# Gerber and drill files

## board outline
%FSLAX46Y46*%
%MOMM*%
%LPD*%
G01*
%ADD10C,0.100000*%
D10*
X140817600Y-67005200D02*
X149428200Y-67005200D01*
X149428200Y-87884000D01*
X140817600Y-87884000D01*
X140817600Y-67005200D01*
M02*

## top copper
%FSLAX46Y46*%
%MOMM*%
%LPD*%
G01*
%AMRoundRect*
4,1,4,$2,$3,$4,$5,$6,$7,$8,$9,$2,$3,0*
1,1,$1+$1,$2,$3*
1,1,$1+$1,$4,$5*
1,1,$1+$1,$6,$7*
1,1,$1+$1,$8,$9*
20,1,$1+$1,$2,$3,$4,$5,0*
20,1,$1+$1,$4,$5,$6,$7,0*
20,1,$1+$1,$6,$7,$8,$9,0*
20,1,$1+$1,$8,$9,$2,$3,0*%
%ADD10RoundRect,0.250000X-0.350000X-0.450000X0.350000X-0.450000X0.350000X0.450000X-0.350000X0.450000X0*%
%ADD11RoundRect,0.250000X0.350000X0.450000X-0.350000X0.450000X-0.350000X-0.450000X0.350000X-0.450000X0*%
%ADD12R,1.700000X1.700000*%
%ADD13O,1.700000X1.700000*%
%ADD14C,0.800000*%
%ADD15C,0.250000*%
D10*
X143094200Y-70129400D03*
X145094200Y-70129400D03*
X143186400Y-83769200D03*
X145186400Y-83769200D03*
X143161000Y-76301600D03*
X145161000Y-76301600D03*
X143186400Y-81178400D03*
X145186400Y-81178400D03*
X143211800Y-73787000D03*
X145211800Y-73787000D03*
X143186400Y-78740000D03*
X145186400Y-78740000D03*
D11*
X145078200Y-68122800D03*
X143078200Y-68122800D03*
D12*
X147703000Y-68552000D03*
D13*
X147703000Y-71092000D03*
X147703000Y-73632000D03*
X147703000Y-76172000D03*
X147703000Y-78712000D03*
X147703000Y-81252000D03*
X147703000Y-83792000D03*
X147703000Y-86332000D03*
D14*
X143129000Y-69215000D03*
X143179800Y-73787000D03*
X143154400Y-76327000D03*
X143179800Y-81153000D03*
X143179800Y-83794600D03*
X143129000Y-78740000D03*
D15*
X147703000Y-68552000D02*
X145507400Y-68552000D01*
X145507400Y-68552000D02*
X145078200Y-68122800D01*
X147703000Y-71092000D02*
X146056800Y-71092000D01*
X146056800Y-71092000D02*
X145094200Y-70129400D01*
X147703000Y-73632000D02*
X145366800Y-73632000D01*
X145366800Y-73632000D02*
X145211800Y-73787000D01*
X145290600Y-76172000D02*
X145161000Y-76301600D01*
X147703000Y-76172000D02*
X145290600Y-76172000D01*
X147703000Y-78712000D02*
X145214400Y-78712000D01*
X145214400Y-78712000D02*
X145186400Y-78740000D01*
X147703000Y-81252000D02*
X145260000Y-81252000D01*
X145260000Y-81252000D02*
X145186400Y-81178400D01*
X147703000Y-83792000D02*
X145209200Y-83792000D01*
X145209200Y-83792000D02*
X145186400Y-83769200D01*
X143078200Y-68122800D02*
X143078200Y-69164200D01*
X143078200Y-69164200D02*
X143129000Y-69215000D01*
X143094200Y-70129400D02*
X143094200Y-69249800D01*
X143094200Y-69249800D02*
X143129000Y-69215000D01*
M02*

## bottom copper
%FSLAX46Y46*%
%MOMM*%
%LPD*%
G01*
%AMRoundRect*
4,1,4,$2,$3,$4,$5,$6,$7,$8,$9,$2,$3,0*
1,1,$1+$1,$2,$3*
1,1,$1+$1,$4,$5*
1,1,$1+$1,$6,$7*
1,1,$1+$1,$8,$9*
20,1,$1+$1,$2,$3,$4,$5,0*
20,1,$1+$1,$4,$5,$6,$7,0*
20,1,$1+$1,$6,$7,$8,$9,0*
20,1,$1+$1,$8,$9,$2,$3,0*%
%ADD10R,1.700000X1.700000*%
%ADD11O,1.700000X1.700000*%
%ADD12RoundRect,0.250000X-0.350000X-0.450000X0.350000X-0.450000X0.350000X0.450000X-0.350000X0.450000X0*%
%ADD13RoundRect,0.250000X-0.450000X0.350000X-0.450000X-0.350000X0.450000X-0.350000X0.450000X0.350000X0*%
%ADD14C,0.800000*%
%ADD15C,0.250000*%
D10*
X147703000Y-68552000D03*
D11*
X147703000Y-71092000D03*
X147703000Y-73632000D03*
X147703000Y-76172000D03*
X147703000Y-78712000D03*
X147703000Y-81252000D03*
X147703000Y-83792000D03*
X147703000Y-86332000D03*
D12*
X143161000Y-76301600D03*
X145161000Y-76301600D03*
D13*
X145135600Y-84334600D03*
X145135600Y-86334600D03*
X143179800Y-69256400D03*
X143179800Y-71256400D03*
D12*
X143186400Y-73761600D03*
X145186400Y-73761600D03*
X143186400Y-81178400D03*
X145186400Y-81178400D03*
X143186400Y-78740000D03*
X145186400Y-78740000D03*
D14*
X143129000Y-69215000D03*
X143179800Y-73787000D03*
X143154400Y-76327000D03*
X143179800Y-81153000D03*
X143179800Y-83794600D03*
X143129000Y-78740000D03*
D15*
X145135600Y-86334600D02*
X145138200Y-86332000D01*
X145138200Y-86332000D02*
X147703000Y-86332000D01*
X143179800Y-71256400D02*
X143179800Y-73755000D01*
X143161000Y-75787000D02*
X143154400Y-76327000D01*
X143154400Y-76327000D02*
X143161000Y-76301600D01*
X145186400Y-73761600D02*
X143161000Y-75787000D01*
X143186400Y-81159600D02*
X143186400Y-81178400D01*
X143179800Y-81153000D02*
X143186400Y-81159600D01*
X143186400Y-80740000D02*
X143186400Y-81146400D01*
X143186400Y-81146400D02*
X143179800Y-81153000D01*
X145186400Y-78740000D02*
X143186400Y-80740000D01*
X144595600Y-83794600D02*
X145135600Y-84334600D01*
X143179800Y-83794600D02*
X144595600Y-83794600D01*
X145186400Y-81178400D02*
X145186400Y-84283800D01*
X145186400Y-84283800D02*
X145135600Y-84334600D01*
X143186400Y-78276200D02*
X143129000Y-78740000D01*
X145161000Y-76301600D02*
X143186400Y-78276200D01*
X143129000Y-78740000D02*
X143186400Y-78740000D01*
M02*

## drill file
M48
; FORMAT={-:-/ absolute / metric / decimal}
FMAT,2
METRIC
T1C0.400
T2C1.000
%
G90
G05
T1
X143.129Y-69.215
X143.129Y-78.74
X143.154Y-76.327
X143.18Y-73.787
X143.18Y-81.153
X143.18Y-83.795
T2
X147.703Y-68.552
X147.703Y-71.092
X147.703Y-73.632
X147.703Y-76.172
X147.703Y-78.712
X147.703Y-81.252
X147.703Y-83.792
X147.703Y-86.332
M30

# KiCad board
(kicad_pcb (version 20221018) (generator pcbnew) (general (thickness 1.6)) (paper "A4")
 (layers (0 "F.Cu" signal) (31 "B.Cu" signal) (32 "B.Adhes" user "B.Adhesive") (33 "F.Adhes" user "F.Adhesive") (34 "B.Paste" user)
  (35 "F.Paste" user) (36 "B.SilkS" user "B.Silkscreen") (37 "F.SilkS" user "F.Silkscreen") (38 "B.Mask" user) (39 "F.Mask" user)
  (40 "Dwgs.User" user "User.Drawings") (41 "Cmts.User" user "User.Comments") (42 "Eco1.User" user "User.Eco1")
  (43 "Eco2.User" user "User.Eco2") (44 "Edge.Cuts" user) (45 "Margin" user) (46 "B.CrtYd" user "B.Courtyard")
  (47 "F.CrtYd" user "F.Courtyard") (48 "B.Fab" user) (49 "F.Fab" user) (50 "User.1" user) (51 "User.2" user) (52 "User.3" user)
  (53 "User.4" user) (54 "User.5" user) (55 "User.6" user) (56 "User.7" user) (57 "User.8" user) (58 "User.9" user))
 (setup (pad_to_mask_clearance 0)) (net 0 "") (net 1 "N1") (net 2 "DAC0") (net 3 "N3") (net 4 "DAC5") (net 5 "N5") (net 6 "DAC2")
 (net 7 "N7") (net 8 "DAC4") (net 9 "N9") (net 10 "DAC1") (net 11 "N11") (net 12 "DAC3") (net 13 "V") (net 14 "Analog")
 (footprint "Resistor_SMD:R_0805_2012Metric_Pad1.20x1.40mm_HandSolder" (layer "F.Cu") (at 144.0942 70.1294)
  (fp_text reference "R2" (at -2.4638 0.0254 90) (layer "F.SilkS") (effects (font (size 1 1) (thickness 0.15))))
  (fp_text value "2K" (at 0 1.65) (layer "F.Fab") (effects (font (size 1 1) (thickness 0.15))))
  (pad "1" smd roundrect (at -1 0) (size 1.2 1.4) (layers "F.Cu" "F.Paste" "F.Mask") (roundrect_rratio 0.208333) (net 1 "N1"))
  (pad "2" smd roundrect (at 1 0) (size 1.2 1.4) (layers "F.Cu" "F.Paste" "F.Mask") (roundrect_rratio 0.208333) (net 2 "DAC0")))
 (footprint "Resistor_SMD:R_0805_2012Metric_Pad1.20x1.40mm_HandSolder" (layer "F.Cu") (at 144.1864 83.7692)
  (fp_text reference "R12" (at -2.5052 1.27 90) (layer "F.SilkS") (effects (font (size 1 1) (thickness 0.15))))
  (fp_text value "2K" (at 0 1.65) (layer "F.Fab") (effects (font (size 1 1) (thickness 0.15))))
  (pad "1" smd roundrect (at -1 0) (size 1.2 1.4) (layers "F.Cu" "F.Paste" "F.Mask") (roundrect_rratio 0.208333) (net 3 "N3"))
  (pad "2" smd roundrect (at 1 0) (size 1.2 1.4) (layers "F.Cu" "F.Paste" "F.Mask") (roundrect_rratio 0.208333) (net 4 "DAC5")))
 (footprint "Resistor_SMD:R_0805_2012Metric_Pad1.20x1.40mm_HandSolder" (layer "F.Cu") (at 144.161 76.3016)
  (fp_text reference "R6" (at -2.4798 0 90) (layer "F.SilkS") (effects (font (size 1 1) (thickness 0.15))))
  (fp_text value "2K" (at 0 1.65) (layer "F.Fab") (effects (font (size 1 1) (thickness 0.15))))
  (pad "1" smd roundrect (at -1 0) (size 1.2 1.4) (layers "F.Cu" "F.Paste" "F.Mask") (roundrect_rratio 0.208333) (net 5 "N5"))
  (pad "2" smd roundrect (at 1 0) (size 1.2 1.4) (layers "F.Cu" "F.Paste" "F.Mask") (roundrect_rratio 0.208333) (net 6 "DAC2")))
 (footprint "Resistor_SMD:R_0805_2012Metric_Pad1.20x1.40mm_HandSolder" (layer "F.Cu") (at 144.1864 81.1784)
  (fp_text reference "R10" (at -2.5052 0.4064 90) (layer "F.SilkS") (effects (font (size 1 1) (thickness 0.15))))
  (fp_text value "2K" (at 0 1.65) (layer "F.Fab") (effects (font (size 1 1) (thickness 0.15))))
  (pad "1" smd roundrect (at -1 0) (size 1.2 1.4) (layers "F.Cu" "F.Paste" "F.Mask") (roundrect_rratio 0.208333) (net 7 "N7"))
  (pad "2" smd roundrect (at 1 0) (size 1.2 1.4) (layers "F.Cu" "F.Paste" "F.Mask") (roundrect_rratio 0.208333) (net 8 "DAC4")))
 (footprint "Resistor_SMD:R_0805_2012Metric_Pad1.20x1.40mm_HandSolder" (layer "F.Cu") (at 144.2118 73.787)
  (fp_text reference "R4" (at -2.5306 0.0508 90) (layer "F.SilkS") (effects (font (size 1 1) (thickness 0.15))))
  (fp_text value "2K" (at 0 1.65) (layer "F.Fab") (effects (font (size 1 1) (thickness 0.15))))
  (pad "1" smd roundrect (at -1 0) (size 1.2 1.4) (layers "F.Cu" "F.Paste" "F.Mask") (roundrect_rratio 0.208333) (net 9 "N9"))
  (pad "2" smd roundrect (at 1 0) (size 1.2 1.4) (layers "F.Cu" "F.Paste" "F.Mask") (roundrect_rratio 0.208333) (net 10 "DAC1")))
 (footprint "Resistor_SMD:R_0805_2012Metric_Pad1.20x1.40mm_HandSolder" (layer "F.Cu") (at 144.1864 78.74)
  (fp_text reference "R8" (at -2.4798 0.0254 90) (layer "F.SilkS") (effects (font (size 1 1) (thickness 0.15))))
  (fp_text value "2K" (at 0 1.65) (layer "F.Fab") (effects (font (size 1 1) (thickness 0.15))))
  (pad "1" smd roundrect (at -1 0) (size 1.2 1.4) (layers "F.Cu" "F.Paste" "F.Mask") (roundrect_rratio 0.208333) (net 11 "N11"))
  (pad "2" smd roundrect (at 1 0) (size 1.2 1.4) (layers "F.Cu" "F.Paste" "F.Mask") (roundrect_rratio 0.208333) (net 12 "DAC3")))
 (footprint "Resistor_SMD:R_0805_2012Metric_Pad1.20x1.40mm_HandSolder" (layer "F.Cu") (at 144.0782 68.1228 180)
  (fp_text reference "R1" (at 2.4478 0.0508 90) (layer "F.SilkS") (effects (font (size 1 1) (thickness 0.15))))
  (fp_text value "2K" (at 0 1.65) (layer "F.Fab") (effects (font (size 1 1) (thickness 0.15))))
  (pad "1" smd roundrect (at -1 0 180) (size 1.2 1.4) (layers "F.Cu" "F.Paste" "F.Mask") (roundrect_rratio 0.208333) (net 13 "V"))
  (pad "2" smd roundrect (at 1 0 180) (size 1.2 1.4) (layers "F.Cu" "F.Paste" "F.Mask") (roundrect_rratio 0.208333) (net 1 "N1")))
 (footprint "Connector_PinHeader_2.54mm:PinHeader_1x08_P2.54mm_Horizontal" (layer "F.Cu") (at 147.703 68.552)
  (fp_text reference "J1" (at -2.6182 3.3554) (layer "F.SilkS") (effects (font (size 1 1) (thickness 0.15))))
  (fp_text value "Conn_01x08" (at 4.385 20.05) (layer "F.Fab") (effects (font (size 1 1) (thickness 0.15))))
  (pad "1" thru_hole rect (at 0 0) (size 1.7 1.7) (drill 1) (layers "*.Cu" "*.Mask") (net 13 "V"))
  (pad "2" thru_hole oval (at 0 2.54) (size 1.7 1.7) (drill 1) (layers "*.Cu" "*.Mask") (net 2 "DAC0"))
  (pad "3" thru_hole oval (at 0 5.08) (size 1.7 1.7) (drill 1) (layers "*.Cu" "*.Mask") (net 10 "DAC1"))
  (pad "4" thru_hole oval (at 0 7.62) (size 1.7 1.7) (drill 1) (layers "*.Cu" "*.Mask") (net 6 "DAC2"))
  (pad "5" thru_hole oval (at 0 10.16) (size 1.7 1.7) (drill 1) (layers "*.Cu" "*.Mask") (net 12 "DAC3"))
  (pad "6" thru_hole oval (at 0 12.7) (size 1.7 1.7) (drill 1) (layers "*.Cu" "*.Mask") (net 8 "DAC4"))
  (pad "7" thru_hole oval (at 0 15.24) (size 1.7 1.7) (drill 1) (layers "*.Cu" "*.Mask") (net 4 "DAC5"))
  (pad "8" thru_hole oval (at 0 17.78) (size 1.7 1.7) (drill 1) (layers "*.Cu" "*.Mask") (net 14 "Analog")))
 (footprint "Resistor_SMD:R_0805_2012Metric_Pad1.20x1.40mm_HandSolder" (layer "B.Cu") (at 144.161 76.3016)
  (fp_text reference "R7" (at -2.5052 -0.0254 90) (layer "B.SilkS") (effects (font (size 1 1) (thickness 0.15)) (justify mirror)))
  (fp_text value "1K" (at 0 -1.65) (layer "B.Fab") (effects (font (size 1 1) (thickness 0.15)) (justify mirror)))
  (pad "1" smd roundrect (at -1 0) (size 1.2 1.4) (layers "B.Cu" "B.Paste" "B.Mask") (roundrect_rratio 0.208333) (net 5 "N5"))
  (pad "2" smd roundrect (at 1 0) (size 1.2 1.4) (layers "B.Cu" "B.Paste" "B.Mask") (roundrect_rratio 0.208333) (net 11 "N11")))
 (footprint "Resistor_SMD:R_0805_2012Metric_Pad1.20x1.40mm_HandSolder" (layer "B.Cu") (at 145.1356 85.3346 -90)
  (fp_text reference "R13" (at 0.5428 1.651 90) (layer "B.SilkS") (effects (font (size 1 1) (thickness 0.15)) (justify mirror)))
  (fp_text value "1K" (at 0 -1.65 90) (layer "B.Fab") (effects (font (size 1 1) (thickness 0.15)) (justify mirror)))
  (pad "1" smd roundrect (at -1 0 270) (size 1.2 1.4) (layers "B.Cu" "B.Paste" "B.Mask") (roundrect_rratio 0.208333) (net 3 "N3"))
  (pad "2" smd roundrect (at 1 0 270) (size 1.2 1.4) (layers "B.Cu" "B.Paste" "B.Mask") (roundrect_rratio 0.208333) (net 14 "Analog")))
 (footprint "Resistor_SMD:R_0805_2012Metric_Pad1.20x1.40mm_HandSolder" (layer "B.Cu") (at 143.1798 70.2564 -90)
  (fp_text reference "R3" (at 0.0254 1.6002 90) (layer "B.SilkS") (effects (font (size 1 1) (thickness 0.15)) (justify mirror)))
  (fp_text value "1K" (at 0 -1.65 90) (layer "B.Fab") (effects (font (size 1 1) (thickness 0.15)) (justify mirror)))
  (pad "1" smd roundrect (at -1 0 270) (size 1.2 1.4) (layers "B.Cu" "B.Paste" "B.Mask") (roundrect_rratio 0.208333) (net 1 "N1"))
  (pad "2" smd roundrect (at 1 0 270) (size 1.2 1.4) (layers "B.Cu" "B.Paste" "B.Mask") (roundrect_rratio 0.208333) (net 9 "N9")))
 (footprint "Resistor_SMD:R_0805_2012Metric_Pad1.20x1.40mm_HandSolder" (layer "B.Cu") (at 144.1864 73.7616)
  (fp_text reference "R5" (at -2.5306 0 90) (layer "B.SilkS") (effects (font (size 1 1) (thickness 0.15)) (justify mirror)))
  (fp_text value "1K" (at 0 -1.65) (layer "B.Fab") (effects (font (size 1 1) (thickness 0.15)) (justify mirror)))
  (pad "1" smd roundrect (at -1 0) (size 1.2 1.4) (layers "B.Cu" "B.Paste" "B.Mask") (roundrect_rratio 0.208333) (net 9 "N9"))
  (pad "2" smd roundrect (at 1 0) (size 1.2 1.4) (layers "B.Cu" "B.Paste" "B.Mask") (roundrect_rratio 0.208333) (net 5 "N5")))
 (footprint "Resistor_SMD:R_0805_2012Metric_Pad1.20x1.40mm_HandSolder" (layer "B.Cu") (at 144.1864 81.1784)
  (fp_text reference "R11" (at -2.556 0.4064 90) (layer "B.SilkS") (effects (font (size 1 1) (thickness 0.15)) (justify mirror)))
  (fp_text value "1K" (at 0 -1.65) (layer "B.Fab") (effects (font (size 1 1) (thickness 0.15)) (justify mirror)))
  (pad "1" smd roundrect (at -1 0) (size 1.2 1.4) (layers "B.Cu" "B.Paste" "B.Mask") (roundrect_rratio 0.208333) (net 7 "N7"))
  (pad "2" smd roundrect (at 1 0) (size 1.2 1.4) (layers "B.Cu" "B.Paste" "B.Mask") (roundrect_rratio 0.208333) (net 3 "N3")))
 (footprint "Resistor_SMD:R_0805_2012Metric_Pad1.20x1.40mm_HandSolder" (layer "B.Cu") (at 144.1864 78.74)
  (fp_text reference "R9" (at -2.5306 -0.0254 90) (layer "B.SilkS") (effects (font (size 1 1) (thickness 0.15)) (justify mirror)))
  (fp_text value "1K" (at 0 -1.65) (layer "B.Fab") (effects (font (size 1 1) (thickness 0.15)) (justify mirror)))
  (pad "1" smd roundrect (at -1 0) (size 1.2 1.4) (layers "B.Cu" "B.Paste" "B.Mask") (roundrect_rratio 0.208333) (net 11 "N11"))
  (pad "2" smd roundrect (at 1 0) (size 1.2 1.4) (layers "B.Cu" "B.Paste" "B.Mask") (roundrect_rratio 0.208333) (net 7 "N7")))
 (gr_rect (start 140.8176 67.0052) (end 149.4282 87.884) (stroke (width 0.1) (type default)) (fill none) (layer "Edge.Cuts"))
 (segment (start 147.703 68.552) (end 145.5074 68.552) (width 0.25) (layer "F.Cu") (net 13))
 (segment (start 145.5074 68.552) (end 145.0782 68.1228) (width 0.25) (layer "F.Cu") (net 13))
 (segment (start 147.703 71.092) (end 146.0568 71.092) (width 0.25) (layer "F.Cu") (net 2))
 (segment (start 146.0568 71.092) (end 145.0942 70.1294) (width 0.25) (layer "F.Cu") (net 2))
 (segment (start 147.703 73.632) (end 145.3668 73.632) (width 0.25) (layer "F.Cu") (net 10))
 (segment (start 145.3668 73.632) (end 145.2118 73.787) (width 0.25) (layer "F.Cu") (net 10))
 (segment (start 145.2906 76.172) (end 145.161 76.3016) (width 0.25) (layer "F.Cu") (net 6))
 (segment (start 147.703 76.172) (end 145.2906 76.172) (width 0.25) (layer "F.Cu") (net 6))
 (segment (start 147.703 78.712) (end 145.2144 78.712) (width 0.25) (layer "F.Cu") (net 12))
 (segment (start 145.2144 78.712) (end 145.1864 78.74) (width 0.25) (layer "F.Cu") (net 12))
 (segment (start 147.703 81.252) (end 145.26 81.252) (width 0.25) (layer "F.Cu") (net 8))
 (segment (start 145.26 81.252) (end 145.1864 81.1784) (width 0.25) (layer "F.Cu") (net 8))
 (segment (start 147.703 83.792) (end 145.2092 83.792) (width 0.25) (layer "F.Cu") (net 4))
 (segment (start 145.2092 83.792) (end 145.1864 83.7692) (width 0.25) (layer "F.Cu") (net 4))
 (segment (start 145.1356 86.3346) (end 145.1382 86.332) (width 0.25) (layer "B.Cu") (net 14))
 (segment (start 145.1382 86.332) (end 147.703 86.332) (width 0.25) (layer "B.Cu") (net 14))
 (segment (start 143.0782 68.1228) (end 143.0782 69.1642) (width 0.25) (layer "F.Cu") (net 1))
 (segment (start 143.0782 69.1642) (end 143.129 69.215) (width 0.25) (layer "F.Cu") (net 1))
 (segment (start 143.0942 70.1294) (end 143.0942 69.2498) (width 0.25) (layer "F.Cu") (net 1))
 (segment (start 143.0942 69.2498) (end 143.129 69.215) (width 0.25) (layer "F.Cu") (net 1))
 (via (at 143.129 69.215) (size 0.8) (drill 0.4) (layers "F.Cu" "B.Cu") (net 1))
 (via (at 143.1798 73.787) (size 0.8) (drill 0.4) (layers "F.Cu" "B.Cu") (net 9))
 (segment (start 143.1798 71.2564) (end 143.1798 73.755) (width 0.25) (layer "B.Cu") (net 9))
 (via (at 143.1544 76.327) (size 0.8) (drill 0.4) (layers "F.Cu" "B.Cu") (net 5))
 (segment (start 143.161 75.787) (end 143.1544 76.327) (width 0.25) (layer "B.Cu") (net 5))
 (segment (start 143.1544 76.327) (end 143.161 76.3016) (width 0.25) (layer "B.Cu") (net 5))
 (segment (start 145.1864 73.7616) (end 143.161 75.787) (width 0.25) (layer "B.Cu") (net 5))
 (via (at 143.1798 81.153) (size 0.8) (drill 0.4) (layers "F.Cu" "B.Cu") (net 7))
 (segment (start 143.1864 81.1596) (end 143.1864 81.1784) (width 0.25) (layer "B.Cu") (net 7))
 (segment (start 143.1798 81.153) (end 143.1864 81.1596) (width 0.25) (layer "B.Cu") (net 7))
 (segment (start 143.1864 80.74) (end 143.1864 81.1464) (width 0.25) (layer "B.Cu") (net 7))
 (segment (start 143.1864 81.1464) (end 143.1798 81.153) (width 0.25) (layer "B.Cu") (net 7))
 (segment (start 145.1864 78.74) (end 143.1864 80.74) (width 0.25) (layer "B.Cu") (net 7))
 (via (at 143.1798 83.7946) (size 0.8) (drill 0.4) (layers "F.Cu" "B.Cu") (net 3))
 (segment (start 144.5956 83.7946) (end 145.1356 84.3346) (width 0.25) (layer "B.Cu") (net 3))
 (segment (start 143.1798 83.7946) (end 144.5956 83.7946) (width 0.25) (layer "B.Cu") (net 3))
 (segment (start 145.1864 81.1784) (end 145.1864 84.2838) (width 0.25) (layer "B.Cu") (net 3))
 (segment (start 145.1864 84.2838) (end 145.1356 84.3346) (width 0.25) (layer "B.Cu") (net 3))
 (via (at 143.129 78.74) (size 0.8) (drill 0.4) (layers "F.Cu" "B.Cu") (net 11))
 (segment (start 143.1864 78.2762) (end 143.129 78.74) (width 0.25) (layer "B.Cu") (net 11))
 (segment (start 145.161 76.3016) (end 143.1864 78.2762) (width 0.25) (layer "B.Cu") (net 11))
 (segment (start 143.129 78.74) (end 143.1864 78.74) (width 0.25) (layer "B.Cu") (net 11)))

